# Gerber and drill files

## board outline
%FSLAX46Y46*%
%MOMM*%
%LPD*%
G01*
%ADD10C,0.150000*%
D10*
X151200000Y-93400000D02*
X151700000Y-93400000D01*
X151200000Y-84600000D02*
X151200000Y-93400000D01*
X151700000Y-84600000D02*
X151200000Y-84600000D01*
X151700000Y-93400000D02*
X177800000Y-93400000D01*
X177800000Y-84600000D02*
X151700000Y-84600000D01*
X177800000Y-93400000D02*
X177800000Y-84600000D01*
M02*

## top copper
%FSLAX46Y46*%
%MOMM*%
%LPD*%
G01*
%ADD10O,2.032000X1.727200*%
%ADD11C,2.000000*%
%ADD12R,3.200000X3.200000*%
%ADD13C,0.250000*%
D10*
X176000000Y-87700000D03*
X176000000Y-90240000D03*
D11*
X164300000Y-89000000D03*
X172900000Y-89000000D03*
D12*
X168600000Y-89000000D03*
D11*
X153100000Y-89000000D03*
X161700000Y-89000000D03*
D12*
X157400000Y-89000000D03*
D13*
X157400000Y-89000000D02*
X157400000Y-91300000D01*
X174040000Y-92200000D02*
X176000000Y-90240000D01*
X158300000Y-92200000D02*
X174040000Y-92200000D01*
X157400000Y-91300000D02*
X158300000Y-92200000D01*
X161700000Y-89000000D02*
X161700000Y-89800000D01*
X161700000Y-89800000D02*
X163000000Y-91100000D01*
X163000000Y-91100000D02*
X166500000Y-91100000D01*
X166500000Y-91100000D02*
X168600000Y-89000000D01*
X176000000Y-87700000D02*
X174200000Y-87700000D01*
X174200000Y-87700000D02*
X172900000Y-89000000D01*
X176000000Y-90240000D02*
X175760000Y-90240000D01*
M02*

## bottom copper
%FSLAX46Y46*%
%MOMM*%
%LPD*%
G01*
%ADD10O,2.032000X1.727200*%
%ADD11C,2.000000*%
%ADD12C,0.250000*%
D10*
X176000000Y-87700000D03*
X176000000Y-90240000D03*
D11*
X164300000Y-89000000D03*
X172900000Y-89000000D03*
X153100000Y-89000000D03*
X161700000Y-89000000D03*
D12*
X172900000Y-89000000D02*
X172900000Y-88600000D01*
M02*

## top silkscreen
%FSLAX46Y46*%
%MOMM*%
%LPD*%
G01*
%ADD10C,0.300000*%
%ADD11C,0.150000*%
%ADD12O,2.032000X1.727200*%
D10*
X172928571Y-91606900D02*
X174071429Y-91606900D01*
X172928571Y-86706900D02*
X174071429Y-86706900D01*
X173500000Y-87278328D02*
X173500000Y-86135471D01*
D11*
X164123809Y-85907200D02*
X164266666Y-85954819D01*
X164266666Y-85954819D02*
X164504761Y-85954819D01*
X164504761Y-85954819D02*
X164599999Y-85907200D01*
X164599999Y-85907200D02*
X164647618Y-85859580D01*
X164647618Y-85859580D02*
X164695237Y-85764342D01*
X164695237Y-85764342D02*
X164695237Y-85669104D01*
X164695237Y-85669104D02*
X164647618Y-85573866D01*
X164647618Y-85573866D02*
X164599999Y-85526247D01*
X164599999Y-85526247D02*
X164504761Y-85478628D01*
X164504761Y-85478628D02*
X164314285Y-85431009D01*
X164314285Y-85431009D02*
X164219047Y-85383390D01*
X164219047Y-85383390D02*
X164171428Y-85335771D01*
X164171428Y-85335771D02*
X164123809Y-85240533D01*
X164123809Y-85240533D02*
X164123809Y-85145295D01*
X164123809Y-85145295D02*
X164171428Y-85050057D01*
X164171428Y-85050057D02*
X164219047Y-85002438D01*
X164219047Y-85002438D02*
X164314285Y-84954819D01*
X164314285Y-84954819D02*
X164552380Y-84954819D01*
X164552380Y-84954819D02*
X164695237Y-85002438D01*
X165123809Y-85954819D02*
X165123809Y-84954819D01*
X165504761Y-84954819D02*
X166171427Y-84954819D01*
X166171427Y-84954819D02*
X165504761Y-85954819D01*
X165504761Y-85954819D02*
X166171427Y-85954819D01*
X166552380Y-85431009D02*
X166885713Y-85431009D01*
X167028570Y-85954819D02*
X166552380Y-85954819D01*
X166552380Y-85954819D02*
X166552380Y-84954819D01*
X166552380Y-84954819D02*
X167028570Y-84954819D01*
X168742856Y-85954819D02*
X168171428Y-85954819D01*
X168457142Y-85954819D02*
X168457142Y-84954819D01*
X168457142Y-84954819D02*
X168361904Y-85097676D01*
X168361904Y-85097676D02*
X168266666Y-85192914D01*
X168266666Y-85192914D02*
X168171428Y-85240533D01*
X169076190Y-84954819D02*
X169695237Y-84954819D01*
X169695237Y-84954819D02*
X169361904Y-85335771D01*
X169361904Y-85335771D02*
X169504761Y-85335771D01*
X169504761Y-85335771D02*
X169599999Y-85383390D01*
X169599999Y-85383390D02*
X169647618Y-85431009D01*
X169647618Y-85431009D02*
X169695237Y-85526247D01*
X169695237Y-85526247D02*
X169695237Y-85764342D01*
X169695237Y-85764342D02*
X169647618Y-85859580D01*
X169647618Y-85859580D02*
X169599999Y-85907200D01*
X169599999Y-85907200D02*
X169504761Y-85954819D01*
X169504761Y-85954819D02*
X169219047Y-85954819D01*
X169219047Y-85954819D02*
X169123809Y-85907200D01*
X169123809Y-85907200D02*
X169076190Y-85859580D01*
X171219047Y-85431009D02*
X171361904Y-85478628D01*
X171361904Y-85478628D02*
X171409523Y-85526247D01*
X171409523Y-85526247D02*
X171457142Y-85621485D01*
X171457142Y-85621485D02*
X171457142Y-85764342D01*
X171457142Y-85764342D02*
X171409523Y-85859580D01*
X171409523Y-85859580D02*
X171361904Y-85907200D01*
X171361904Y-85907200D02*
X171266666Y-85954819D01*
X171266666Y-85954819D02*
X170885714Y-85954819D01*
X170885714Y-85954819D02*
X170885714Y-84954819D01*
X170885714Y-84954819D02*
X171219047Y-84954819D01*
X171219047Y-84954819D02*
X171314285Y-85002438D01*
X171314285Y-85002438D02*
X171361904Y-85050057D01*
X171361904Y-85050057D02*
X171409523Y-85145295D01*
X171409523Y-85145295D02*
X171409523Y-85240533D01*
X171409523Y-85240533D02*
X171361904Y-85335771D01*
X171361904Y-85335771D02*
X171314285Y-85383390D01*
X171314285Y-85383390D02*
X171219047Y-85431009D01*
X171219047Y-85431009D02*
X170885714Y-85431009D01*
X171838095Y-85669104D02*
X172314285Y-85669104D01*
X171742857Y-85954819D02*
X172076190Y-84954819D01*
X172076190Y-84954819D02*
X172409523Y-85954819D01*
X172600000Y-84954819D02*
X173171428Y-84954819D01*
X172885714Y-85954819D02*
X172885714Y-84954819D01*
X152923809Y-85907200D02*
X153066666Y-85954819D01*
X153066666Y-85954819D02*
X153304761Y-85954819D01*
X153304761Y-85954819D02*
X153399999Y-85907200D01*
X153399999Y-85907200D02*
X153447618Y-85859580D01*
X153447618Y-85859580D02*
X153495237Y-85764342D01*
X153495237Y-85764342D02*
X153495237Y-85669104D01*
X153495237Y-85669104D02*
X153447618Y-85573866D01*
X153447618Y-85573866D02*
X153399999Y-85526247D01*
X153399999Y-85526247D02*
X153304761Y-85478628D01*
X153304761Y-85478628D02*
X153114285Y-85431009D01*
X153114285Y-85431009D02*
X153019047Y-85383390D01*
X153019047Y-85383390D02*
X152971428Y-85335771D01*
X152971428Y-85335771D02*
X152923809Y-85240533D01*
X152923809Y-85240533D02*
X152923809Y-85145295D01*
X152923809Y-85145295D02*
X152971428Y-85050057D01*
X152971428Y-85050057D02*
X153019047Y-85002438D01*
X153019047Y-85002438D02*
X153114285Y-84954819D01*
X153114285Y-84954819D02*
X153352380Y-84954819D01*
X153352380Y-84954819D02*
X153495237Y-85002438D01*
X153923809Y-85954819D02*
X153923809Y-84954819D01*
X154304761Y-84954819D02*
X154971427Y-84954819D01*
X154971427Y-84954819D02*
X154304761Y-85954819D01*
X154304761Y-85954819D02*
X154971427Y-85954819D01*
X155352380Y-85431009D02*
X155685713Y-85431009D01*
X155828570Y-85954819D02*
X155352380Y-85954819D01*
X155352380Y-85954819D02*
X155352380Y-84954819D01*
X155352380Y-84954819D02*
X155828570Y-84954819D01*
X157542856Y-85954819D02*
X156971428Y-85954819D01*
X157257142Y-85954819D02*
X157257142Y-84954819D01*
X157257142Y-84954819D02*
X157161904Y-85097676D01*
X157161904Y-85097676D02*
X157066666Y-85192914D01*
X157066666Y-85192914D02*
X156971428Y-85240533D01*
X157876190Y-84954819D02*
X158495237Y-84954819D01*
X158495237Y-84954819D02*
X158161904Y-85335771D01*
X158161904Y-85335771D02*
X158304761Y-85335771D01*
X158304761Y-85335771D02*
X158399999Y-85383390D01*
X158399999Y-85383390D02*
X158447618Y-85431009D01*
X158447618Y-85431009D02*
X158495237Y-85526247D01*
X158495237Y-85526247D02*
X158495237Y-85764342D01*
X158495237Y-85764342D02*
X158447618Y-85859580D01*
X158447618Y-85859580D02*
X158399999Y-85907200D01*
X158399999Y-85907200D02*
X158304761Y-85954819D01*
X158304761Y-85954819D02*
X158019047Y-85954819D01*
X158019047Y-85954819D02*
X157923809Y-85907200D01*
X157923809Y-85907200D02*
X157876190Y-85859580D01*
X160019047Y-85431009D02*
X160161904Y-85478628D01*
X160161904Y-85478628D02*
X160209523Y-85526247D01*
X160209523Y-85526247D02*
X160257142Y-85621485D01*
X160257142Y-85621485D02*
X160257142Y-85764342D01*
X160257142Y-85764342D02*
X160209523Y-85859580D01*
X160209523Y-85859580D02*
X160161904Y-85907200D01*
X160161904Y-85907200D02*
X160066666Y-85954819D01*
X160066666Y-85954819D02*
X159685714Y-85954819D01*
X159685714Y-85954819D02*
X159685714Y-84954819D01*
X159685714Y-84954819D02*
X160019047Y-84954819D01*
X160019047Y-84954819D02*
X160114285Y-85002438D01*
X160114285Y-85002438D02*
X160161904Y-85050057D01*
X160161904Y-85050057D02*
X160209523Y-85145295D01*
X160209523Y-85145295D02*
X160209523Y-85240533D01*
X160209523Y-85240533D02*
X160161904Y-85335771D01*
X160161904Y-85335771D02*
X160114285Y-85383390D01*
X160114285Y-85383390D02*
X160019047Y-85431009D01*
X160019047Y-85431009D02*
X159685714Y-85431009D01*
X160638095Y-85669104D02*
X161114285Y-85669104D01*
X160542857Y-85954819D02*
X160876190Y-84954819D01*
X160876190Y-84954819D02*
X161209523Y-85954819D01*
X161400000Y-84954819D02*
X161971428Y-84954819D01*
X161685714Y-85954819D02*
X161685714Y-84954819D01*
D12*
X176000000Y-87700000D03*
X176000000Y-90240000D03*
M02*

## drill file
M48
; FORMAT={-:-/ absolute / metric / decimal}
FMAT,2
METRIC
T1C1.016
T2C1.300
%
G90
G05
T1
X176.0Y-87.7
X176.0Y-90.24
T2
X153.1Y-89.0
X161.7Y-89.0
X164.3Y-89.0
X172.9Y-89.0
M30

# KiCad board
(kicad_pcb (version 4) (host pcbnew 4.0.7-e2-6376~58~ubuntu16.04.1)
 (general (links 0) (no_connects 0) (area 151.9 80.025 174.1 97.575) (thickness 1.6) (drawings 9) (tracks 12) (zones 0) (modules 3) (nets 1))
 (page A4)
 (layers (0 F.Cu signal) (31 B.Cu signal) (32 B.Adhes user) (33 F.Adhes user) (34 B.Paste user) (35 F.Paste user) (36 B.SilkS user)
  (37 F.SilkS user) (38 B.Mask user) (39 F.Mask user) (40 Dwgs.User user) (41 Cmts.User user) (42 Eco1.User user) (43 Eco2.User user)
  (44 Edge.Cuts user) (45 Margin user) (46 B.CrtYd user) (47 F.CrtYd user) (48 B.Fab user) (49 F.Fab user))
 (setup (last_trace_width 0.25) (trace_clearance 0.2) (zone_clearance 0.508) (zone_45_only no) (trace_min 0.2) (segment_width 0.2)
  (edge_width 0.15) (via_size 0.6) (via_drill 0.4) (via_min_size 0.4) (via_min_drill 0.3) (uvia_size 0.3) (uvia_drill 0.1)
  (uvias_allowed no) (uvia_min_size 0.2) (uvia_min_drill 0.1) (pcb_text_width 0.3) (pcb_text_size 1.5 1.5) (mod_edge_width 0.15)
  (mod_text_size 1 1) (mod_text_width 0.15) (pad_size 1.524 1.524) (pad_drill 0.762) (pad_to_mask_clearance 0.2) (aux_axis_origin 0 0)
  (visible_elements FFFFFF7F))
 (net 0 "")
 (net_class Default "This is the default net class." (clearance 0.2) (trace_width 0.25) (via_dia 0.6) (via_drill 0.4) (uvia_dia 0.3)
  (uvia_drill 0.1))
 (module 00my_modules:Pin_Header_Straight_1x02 (layer F.Cu) (at 176 87.7)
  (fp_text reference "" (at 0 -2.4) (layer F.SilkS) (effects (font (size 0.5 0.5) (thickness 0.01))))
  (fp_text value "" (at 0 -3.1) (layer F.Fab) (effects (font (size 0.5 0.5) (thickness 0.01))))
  (pad 1 thru_hole oval (at 0 0) (size 2.032 1.7272) (drill 1.016) (layers *.Cu *.Mask F.SilkS))
  (pad 2 thru_hole oval (at 0 2.54) (size 2.032 1.7272) (drill 1.016) (layers *.Cu *.Mask F.SilkS)))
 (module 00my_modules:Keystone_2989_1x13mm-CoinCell (layer F.Cu) (at 168.6 89)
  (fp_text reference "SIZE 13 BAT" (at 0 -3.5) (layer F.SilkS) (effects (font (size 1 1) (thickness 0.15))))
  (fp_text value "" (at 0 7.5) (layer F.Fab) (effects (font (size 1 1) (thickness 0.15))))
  (pad 1 thru_hole circle (at -4.3 0) (size 2 2) (drill 1.3) (layers *.Cu *.Mask))
  (pad 1 thru_hole circle (at 4.3 0) (size 2 2) (drill 1.3) (layers *.Cu *.Mask))
  (pad 2 smd rect (at 0 0) (size 3.2 3.2) (layers F.Cu F.Mask)))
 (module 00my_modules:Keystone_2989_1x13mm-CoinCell (layer F.Cu) (at 157.4 89)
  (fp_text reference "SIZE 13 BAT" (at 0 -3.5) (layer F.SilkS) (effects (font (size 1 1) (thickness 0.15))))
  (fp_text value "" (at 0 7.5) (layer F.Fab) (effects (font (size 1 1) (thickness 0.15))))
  (pad 1 thru_hole circle (at -4.3 0) (size 2 2) (drill 1.3) (layers *.Cu *.Mask))
  (pad 1 thru_hole circle (at 4.3 0) (size 2 2) (drill 1.3) (layers *.Cu *.Mask))
  (pad 2 smd rect (at 0 0) (size 3.2 3.2) (layers F.Cu F.Mask)))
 (gr_line (start 151.2 93.4) (end 151.7 93.4) (angle 90) (layer Edge.Cuts) (width 0.15))
 (gr_line (start 151.2 84.6) (end 151.2 93.4) (angle 90) (layer Edge.Cuts) (width 0.15))
 (gr_line (start 151.7 84.6) (end 151.2 84.6) (angle 90) (layer Edge.Cuts) (width 0.15))
 (gr_line (start 151.7 93.4) (end 177.8 93.4) (angle 90) (layer Edge.Cuts) (width 0.15))
 (gr_line (start 177.8 84.6) (end 151.7 84.6) (angle 90) (layer Edge.Cuts) (width 0.15))
 (gr_line (start 177.8 93.4) (end 177.8 84.6) (angle 90) (layer Edge.Cuts) (width 0.15))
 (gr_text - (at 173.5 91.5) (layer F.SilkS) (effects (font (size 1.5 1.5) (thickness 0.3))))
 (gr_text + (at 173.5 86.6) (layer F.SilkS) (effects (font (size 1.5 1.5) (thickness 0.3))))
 (segment (start 157.4 89) (end 157.4 91.3) (width 0.25) (layer F.Cu) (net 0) (status 400000))
 (segment (start 174.04 92.2) (end 176 90.24) (width 0.25) (layer F.Cu) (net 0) (status 800000))
 (segment (start 158.3 92.2) (end 174.04 92.2) (width 0.25) (layer F.Cu) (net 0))
 (segment (start 157.4 91.3) (end 158.3 92.2) (width 0.25) (layer F.Cu) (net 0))
 (segment (start 161.7 89) (end 161.7 89.8) (width 0.25) (layer F.Cu) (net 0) (status C00000))
 (segment (start 161.7 89.8) (end 163 91.1) (width 0.25) (layer F.Cu) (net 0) (status 400000))
 (segment (start 163 91.1) (end 166.5 91.1) (width 0.25) (layer F.Cu) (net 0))
 (segment (start 166.5 91.1) (end 168.6 89) (width 0.25) (layer F.Cu) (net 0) (status 800000))
 (segment (start 176 87.7) (end 174.2 87.7) (width 0.25) (layer F.Cu) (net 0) (status 400000))
 (segment (start 174.2 87.7) (end 172.9 89) (width 0.25) (layer F.Cu) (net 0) (status 800000))
 (segment (start 176 90.24) (end 175.76 90.24) (width 0.25) (layer F.Cu) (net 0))
 (segment (start 172.9 89) (end 172.9 88.6) (width 0.25) (layer B.Cu) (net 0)))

